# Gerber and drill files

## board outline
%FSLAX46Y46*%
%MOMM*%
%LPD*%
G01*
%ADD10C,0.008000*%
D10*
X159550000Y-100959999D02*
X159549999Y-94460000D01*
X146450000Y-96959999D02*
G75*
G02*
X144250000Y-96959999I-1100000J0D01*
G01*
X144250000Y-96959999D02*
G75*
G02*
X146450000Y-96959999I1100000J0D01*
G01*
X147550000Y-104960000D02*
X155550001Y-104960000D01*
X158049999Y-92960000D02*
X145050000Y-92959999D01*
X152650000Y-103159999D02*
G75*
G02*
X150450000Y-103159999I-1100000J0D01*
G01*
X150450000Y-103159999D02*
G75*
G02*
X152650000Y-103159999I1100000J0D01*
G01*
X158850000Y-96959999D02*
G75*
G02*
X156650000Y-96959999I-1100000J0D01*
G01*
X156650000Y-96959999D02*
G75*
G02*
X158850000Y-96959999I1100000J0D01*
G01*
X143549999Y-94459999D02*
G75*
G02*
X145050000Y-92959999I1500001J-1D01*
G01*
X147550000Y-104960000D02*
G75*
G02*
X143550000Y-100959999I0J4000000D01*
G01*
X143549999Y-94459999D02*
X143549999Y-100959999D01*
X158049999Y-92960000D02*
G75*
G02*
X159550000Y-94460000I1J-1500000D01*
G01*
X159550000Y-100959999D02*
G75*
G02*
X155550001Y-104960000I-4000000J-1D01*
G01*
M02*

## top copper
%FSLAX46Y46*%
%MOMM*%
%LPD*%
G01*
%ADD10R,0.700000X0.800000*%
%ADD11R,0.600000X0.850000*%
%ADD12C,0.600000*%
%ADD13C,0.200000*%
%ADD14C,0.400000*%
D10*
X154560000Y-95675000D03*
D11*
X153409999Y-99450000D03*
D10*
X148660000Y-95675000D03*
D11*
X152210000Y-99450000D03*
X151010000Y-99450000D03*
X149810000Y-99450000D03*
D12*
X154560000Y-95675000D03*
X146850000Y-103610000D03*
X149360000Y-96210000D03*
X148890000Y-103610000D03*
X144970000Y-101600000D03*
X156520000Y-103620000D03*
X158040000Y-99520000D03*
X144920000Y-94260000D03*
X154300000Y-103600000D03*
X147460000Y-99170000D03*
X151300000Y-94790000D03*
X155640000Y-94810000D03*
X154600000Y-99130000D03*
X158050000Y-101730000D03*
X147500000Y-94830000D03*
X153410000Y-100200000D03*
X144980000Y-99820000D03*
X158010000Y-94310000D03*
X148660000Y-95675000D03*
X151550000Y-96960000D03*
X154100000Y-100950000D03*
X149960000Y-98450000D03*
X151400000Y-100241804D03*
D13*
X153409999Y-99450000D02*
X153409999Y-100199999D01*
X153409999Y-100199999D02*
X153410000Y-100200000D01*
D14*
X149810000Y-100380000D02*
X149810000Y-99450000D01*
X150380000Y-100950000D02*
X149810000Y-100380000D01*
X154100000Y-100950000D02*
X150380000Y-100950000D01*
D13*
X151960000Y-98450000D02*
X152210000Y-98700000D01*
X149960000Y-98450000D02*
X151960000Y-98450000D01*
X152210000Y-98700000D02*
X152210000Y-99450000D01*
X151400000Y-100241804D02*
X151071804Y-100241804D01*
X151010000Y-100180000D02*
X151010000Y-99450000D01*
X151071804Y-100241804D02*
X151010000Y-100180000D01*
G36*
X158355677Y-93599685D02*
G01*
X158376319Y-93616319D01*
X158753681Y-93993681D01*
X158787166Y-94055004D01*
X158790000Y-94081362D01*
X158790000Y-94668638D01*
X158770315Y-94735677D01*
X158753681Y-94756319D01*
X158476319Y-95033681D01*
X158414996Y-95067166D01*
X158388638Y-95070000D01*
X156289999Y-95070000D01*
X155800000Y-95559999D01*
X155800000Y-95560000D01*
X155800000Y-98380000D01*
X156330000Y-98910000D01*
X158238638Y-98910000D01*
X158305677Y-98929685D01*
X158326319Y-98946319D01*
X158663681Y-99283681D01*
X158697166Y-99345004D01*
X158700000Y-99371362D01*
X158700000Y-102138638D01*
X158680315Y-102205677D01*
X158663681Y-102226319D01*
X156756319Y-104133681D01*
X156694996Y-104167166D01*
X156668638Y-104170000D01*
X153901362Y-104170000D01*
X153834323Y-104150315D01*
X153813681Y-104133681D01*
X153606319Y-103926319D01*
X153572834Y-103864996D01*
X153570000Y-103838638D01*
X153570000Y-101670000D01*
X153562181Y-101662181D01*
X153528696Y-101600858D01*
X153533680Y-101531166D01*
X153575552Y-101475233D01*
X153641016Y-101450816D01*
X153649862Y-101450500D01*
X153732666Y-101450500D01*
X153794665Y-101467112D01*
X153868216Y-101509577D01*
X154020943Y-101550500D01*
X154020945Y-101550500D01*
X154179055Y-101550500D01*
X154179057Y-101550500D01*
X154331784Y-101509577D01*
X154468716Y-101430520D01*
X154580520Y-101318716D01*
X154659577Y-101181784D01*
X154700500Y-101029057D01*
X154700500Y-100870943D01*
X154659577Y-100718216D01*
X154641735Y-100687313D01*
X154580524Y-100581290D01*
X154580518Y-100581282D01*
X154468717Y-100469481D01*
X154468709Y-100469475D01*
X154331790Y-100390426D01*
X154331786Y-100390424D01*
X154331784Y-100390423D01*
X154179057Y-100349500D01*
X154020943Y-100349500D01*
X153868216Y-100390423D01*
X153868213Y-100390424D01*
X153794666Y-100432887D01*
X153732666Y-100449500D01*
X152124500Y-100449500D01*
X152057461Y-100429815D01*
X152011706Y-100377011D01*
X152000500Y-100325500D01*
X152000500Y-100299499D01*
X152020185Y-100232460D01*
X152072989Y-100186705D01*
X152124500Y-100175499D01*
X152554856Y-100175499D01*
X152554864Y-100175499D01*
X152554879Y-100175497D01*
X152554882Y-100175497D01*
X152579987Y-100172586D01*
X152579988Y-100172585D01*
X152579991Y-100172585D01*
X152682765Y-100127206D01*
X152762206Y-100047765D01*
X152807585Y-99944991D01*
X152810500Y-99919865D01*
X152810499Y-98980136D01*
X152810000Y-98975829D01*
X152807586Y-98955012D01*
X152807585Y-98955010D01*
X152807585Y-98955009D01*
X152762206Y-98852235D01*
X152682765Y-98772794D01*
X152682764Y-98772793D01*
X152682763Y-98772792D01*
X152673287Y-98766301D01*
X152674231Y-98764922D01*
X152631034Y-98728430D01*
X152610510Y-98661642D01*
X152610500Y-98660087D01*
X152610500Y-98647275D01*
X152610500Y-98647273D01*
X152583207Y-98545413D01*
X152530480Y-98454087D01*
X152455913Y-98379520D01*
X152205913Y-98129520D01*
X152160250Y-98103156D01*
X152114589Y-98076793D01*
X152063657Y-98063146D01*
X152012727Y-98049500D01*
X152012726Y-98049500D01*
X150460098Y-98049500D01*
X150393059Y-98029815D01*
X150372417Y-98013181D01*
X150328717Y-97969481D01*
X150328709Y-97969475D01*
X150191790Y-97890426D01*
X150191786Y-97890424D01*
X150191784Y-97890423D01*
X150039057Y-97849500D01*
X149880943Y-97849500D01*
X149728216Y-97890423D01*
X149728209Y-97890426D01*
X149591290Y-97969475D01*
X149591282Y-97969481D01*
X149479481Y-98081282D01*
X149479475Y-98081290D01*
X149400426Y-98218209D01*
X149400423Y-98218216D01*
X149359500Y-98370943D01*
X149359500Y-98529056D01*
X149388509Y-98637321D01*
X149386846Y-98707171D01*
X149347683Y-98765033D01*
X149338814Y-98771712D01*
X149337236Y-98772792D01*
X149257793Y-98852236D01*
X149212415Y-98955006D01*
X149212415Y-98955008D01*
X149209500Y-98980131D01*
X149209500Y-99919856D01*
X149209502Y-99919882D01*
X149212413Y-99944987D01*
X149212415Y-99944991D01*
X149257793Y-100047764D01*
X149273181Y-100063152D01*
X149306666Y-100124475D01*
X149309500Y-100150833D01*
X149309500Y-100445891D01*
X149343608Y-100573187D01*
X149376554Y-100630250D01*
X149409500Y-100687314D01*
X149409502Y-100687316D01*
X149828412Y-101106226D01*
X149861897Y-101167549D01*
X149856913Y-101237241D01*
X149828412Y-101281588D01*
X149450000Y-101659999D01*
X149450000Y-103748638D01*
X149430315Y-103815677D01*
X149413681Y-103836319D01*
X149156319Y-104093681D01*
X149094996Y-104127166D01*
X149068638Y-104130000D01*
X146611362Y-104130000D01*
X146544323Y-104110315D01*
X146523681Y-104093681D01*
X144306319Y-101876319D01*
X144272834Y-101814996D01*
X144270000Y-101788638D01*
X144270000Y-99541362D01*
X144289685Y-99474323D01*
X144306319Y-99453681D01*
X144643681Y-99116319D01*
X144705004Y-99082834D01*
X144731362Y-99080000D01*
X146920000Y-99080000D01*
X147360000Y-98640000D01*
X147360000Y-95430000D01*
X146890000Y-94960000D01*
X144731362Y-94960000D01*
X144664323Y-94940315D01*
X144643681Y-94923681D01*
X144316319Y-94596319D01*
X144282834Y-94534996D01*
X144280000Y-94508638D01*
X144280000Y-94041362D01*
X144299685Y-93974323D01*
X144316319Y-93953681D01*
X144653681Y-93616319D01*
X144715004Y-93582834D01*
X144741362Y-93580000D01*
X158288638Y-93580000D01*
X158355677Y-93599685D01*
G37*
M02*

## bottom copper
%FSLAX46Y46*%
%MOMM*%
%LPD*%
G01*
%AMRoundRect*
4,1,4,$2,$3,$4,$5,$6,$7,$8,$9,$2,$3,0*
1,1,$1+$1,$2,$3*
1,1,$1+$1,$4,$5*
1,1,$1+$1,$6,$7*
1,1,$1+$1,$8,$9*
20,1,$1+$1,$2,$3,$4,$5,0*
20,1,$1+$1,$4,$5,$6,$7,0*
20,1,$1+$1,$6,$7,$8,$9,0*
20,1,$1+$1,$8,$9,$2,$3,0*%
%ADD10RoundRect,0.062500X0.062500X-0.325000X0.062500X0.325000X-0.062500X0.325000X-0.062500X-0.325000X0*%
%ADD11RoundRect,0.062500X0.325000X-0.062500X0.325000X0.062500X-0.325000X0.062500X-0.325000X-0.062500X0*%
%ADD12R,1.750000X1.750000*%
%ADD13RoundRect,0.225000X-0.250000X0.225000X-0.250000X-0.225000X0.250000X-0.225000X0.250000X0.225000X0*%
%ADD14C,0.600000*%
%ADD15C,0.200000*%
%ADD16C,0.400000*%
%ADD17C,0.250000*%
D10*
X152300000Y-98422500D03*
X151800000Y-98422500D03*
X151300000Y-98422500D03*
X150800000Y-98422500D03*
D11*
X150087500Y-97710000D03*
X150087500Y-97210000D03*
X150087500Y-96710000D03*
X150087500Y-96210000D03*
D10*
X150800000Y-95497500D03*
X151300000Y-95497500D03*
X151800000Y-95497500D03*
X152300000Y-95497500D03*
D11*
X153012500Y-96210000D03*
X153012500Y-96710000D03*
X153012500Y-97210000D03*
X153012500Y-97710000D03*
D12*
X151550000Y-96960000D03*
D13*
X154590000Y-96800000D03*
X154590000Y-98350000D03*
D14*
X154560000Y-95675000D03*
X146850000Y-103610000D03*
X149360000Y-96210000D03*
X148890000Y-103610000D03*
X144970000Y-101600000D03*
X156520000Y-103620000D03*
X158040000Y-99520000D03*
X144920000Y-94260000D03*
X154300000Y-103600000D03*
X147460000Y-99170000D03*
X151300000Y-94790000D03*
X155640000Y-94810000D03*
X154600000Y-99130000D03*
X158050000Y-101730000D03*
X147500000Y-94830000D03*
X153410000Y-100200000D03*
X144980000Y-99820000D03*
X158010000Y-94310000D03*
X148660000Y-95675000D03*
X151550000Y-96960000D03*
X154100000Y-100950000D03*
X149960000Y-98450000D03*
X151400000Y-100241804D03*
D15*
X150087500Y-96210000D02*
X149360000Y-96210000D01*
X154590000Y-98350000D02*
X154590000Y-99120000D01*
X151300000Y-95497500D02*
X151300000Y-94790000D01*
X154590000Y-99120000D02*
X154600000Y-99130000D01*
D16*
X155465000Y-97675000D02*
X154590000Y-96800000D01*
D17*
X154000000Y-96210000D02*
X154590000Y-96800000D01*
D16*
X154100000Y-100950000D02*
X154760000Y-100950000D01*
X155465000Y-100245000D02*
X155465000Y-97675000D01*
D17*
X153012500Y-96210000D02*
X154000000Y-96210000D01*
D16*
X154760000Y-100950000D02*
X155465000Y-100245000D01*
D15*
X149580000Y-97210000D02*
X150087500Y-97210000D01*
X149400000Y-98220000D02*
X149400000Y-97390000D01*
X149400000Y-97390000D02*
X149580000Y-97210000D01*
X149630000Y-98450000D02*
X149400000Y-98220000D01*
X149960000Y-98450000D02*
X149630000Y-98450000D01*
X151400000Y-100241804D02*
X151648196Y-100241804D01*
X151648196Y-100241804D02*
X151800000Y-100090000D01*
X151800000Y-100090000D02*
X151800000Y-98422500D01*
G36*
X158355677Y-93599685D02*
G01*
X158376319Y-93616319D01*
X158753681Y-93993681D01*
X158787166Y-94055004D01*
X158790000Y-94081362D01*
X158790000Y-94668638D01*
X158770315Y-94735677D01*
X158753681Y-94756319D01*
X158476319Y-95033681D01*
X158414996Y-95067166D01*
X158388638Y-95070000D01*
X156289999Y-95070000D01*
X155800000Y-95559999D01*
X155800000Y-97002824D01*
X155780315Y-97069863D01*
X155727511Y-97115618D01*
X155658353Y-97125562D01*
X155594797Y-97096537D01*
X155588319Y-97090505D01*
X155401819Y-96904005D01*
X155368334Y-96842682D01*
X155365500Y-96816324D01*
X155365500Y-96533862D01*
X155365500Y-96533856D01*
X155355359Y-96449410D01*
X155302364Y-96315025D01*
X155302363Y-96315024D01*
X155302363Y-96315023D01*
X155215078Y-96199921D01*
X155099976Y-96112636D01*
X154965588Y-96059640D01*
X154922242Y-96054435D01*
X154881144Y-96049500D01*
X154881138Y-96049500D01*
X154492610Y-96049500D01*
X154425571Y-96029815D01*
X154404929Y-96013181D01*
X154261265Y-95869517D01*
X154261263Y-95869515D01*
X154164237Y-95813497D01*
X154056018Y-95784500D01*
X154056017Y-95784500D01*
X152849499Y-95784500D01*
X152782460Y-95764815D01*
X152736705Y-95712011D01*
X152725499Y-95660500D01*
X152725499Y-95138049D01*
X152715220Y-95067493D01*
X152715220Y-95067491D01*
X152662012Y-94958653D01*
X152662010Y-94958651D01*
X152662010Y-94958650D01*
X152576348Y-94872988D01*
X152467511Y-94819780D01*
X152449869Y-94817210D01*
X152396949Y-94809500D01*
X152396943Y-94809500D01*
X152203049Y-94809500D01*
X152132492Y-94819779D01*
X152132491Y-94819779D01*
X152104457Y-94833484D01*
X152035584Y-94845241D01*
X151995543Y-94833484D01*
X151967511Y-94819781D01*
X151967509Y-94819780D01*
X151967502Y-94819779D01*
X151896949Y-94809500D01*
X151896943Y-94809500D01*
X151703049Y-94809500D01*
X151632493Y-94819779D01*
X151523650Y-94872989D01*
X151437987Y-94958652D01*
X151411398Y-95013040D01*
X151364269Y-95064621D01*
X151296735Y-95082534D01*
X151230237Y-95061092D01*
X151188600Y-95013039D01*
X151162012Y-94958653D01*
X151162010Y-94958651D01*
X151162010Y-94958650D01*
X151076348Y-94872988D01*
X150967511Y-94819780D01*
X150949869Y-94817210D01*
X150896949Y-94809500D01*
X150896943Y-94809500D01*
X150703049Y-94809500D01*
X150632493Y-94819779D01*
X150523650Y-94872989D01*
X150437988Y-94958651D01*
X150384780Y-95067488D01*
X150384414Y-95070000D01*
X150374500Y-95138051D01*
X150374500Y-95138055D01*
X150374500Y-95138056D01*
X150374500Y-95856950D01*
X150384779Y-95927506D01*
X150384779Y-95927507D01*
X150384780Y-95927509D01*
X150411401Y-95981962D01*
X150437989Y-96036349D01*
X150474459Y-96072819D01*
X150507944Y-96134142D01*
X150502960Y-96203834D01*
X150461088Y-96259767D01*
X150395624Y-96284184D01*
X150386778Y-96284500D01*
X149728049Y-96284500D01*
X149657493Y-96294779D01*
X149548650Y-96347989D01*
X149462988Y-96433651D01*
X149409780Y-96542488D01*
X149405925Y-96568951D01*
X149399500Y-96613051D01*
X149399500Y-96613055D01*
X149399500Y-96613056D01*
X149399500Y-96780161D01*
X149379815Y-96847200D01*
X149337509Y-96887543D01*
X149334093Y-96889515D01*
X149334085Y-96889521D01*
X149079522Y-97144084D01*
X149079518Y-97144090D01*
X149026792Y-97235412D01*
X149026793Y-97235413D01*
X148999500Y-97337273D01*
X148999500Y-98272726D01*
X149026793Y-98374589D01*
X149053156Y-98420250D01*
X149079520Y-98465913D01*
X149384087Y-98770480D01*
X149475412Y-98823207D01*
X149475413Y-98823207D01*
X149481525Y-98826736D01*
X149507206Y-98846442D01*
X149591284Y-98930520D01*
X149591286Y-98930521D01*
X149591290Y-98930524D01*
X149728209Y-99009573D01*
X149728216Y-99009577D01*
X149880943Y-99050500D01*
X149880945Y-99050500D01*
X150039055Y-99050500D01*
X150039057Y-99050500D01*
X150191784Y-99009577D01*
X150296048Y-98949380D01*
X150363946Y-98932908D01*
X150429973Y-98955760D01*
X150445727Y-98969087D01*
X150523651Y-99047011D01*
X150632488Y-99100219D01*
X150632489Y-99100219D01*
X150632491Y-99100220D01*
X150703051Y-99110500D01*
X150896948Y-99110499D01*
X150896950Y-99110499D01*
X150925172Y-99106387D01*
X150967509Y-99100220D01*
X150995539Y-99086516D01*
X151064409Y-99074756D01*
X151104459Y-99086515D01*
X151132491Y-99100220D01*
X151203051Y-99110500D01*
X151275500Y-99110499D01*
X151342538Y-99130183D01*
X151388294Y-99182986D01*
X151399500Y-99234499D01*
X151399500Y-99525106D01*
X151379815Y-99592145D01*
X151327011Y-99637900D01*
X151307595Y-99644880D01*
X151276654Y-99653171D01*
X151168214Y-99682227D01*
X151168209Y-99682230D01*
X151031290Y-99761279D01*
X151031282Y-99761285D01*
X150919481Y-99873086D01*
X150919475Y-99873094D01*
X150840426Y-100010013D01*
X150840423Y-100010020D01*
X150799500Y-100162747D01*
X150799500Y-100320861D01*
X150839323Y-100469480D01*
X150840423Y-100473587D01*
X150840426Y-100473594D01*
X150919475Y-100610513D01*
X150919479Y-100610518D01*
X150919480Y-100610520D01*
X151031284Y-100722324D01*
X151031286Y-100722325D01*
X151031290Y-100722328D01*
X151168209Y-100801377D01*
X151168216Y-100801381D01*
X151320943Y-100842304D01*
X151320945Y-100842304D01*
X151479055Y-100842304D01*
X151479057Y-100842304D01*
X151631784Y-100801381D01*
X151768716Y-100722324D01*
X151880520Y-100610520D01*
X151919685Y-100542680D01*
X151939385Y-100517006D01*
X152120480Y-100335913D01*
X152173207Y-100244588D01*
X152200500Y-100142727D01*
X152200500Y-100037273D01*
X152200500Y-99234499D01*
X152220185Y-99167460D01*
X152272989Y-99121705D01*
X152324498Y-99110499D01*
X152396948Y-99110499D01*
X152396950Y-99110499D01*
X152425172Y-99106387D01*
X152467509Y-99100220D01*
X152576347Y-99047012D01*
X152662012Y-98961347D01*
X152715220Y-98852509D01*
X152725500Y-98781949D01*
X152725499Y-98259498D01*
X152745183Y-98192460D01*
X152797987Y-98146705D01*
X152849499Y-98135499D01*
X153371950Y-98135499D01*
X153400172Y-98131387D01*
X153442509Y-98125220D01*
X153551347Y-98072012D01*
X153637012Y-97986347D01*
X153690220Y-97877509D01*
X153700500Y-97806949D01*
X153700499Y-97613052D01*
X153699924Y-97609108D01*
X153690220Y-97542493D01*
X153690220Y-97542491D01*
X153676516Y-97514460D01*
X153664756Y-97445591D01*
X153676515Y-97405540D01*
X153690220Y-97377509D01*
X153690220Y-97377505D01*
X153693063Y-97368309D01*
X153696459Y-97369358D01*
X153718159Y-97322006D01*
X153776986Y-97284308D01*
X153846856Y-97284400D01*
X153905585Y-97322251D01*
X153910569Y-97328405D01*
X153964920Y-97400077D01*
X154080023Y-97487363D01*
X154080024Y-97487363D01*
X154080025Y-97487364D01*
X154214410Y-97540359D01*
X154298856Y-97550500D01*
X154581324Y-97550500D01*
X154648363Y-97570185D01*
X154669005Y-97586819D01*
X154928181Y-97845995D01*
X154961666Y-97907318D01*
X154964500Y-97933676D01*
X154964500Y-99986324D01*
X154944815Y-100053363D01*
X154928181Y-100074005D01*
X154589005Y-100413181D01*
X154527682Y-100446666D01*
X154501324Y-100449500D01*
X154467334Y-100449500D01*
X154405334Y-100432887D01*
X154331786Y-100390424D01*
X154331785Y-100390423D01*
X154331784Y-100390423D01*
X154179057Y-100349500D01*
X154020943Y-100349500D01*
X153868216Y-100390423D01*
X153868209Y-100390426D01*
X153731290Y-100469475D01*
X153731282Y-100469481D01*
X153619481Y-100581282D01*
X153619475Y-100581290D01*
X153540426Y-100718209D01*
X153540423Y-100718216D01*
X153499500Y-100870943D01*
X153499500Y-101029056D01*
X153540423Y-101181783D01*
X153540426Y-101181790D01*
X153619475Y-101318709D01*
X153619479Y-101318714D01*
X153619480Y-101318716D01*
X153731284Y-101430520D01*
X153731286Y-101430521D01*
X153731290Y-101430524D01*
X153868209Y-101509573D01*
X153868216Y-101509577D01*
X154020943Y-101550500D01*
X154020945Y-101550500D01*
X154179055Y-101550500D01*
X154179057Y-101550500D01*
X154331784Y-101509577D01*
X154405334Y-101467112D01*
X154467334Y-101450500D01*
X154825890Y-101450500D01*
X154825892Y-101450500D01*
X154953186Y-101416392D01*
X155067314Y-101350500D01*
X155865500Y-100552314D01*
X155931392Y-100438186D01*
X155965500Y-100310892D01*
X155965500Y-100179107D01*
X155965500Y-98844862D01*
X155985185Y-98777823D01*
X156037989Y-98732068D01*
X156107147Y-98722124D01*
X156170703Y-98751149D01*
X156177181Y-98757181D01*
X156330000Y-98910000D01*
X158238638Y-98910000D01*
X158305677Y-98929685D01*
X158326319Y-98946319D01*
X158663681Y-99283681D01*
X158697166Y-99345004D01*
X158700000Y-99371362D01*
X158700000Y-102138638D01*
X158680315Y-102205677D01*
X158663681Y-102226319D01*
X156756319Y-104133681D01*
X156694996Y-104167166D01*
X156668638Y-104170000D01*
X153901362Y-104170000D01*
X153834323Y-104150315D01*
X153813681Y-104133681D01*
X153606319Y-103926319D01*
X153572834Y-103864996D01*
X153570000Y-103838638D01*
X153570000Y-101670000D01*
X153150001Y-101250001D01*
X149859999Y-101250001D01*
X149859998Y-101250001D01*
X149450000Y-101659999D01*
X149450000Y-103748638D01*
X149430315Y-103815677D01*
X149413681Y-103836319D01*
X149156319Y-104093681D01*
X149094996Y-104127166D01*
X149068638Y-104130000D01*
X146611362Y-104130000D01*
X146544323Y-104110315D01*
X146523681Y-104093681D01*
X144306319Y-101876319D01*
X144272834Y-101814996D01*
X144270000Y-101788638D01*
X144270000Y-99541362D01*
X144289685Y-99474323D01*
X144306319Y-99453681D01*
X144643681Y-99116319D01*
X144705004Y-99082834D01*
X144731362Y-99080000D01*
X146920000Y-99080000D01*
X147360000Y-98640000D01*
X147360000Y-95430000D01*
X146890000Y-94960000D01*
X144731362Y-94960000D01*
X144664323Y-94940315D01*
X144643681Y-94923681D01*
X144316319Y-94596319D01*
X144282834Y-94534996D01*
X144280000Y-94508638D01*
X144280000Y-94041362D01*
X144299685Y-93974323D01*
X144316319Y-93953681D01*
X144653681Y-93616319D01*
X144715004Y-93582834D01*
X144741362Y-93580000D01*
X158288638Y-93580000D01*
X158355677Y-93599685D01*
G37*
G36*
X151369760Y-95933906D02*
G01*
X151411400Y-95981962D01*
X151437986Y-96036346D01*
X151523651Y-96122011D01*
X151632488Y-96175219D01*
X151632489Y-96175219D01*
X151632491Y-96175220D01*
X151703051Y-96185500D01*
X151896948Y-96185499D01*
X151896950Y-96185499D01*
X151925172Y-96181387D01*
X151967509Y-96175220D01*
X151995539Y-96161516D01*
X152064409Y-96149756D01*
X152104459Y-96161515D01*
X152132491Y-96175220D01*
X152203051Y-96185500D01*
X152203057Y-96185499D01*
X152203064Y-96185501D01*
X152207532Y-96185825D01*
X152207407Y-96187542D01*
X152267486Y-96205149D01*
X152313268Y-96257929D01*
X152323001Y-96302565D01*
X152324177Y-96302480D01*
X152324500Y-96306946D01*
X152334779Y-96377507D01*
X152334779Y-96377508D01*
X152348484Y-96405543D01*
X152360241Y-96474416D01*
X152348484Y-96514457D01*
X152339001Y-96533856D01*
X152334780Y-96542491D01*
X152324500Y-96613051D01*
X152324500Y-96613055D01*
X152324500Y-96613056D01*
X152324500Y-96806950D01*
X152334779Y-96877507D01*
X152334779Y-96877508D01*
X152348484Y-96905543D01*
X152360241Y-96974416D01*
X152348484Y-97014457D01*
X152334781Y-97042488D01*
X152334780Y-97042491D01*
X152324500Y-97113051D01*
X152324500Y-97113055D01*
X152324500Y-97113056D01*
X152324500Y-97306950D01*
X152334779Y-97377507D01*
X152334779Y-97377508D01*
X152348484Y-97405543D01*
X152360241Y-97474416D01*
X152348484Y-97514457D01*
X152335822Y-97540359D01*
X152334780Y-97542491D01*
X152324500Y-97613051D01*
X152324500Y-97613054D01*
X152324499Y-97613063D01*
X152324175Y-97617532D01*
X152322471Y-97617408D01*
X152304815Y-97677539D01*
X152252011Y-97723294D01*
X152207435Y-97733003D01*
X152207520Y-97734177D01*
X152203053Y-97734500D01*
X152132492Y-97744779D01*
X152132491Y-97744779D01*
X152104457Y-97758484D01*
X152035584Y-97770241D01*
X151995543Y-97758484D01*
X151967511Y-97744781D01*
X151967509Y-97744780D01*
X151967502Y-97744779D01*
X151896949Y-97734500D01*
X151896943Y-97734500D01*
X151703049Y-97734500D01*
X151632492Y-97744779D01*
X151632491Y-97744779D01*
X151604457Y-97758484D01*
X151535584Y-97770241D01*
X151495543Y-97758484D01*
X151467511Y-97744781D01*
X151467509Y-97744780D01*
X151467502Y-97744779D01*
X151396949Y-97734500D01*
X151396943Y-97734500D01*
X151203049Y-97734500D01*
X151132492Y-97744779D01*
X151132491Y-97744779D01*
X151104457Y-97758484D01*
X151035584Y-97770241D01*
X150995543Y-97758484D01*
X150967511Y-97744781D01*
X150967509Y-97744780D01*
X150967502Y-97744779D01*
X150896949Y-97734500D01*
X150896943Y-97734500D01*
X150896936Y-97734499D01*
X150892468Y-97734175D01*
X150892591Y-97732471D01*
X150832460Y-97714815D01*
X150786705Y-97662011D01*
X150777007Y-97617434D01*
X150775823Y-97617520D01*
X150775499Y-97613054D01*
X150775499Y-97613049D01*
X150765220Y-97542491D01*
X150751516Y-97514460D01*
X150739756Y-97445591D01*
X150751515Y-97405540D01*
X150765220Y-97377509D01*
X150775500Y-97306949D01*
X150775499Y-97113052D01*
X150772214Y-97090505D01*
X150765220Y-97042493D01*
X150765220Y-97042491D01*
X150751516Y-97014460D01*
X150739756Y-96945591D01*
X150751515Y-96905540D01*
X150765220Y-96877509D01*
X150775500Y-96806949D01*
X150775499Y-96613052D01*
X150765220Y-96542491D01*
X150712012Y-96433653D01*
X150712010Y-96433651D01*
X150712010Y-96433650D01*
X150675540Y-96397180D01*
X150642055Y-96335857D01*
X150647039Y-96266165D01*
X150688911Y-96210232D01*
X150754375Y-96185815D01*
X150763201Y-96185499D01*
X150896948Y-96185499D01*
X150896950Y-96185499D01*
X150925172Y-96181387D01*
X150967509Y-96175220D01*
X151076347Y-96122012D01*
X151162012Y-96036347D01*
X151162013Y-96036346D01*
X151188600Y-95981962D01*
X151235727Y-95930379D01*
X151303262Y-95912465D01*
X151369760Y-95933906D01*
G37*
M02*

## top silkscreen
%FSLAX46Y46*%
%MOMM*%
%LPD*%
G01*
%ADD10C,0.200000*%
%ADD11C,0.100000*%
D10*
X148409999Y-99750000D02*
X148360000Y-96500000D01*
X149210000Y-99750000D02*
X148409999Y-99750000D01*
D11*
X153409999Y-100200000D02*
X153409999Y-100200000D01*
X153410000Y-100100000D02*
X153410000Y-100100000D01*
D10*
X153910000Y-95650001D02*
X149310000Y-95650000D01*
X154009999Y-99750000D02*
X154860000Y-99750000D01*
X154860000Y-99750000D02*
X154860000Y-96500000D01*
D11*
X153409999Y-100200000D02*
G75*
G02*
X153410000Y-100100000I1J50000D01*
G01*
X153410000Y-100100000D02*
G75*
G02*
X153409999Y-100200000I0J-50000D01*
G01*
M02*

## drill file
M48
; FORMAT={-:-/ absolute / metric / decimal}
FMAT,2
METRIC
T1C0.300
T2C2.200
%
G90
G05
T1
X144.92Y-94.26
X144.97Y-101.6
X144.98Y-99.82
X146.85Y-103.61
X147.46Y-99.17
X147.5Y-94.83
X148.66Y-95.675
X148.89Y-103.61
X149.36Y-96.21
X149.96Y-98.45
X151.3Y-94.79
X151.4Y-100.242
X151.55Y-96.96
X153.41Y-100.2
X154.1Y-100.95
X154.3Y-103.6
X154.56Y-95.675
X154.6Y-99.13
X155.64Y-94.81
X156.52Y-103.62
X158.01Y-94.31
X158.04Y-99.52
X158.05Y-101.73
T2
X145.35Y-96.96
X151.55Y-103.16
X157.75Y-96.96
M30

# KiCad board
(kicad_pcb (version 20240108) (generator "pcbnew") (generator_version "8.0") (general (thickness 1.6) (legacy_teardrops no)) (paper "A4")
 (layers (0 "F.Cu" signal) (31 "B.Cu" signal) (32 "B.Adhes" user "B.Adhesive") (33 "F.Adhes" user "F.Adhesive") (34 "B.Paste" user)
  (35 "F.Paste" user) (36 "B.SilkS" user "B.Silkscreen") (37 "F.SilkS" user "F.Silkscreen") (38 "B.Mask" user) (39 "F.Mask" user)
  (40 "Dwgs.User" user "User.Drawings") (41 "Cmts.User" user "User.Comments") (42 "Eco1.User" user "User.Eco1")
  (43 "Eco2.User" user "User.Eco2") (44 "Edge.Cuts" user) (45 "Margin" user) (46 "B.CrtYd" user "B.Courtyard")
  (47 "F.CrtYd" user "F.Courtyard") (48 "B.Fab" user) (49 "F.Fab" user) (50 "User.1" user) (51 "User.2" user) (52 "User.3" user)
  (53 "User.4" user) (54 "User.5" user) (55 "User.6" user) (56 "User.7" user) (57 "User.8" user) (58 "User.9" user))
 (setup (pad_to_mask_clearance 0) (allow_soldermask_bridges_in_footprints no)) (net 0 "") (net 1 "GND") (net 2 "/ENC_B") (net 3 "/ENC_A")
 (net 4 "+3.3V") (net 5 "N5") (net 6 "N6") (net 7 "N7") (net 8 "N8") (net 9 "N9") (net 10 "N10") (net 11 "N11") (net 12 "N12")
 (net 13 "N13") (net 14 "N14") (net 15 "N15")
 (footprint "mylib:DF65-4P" (layer "F.Cu") (at 151.585 97.800001 180)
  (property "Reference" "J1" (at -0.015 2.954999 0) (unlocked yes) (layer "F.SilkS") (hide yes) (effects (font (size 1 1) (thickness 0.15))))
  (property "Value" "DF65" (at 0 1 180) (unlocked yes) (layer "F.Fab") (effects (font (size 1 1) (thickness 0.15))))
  (fp_line (start 3.175001 -1.949999) (end 3.225 1.300001) (stroke (width 0.2) (type solid)) (layer "F.SilkS"))
  (fp_line (start 2.375 -1.949999) (end 3.175001 -1.949999) (stroke (width 0.2) (type solid)) (layer "F.SilkS"))
  (fp_line (start -1.824999 -2.399999) (end -1.824999 -2.399999) (stroke (width 0.1) (type solid)) (layer "F.SilkS"))
  (fp_line (start -1.825 -2.299999) (end -1.825 -2.299999) (stroke (width 0.1) (type solid)) (layer "F.SilkS"))
  (fp_line (start -2.325 2.15) (end 2.275 2.150001) (stroke (width 0.2) (type solid)) (layer "F.SilkS"))
  (fp_line (start -2.424999 -1.949999) (end -3.275 -1.949999) (stroke (width 0.2) (type solid)) (layer "F.SilkS"))
  (fp_line (start -3.275 -1.949999) (end -3.275 1.300001) (stroke (width 0.2) (type solid)) (layer "F.SilkS"))
  (fp_arc (start -1.824999 -2.399999) (mid -1.775 -2.349998) (end -1.825 -2.299999) (stroke (width 0.1) (type solid)) (layer "F.SilkS"))
  (fp_arc (start -1.825 -2.299999) (mid -1.875 -2.349999) (end -1.824999 -2.399999) (stroke (width 0.1) (type solid)) (layer "F.SilkS"))
  (pad "1" smd rect (at -2.975 2.125001 180) (size 0.7 0.8) (layers "F.Cu" "F.Paste" "F.Mask") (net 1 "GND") (thermal_bridge_angle 45))
  (pad "1" smd rect (at -1.824999 -1.649999 180) (size 0.6 0.85) (layers "F.Cu" "F.Paste" "F.Mask") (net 1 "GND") (thermal_bridge_angle 45))
  (pad "1" smd rect (at 2.925 2.125001 180) (size 0.7 0.8) (layers "F.Cu" "F.Paste" "F.Mask") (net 1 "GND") (thermal_bridge_angle 45))
  (pad "2" smd rect (at -0.625 -1.649999 180) (size 0.6 0.85) (layers "F.Cu" "F.Paste" "F.Mask") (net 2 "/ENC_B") (thermal_bridge_angle 45))
  (pad "3" smd rect (at 0.575 -1.649999 180) (size 0.6 0.85) (layers "F.Cu" "F.Paste" "F.Mask") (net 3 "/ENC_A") (thermal_bridge_angle 45))
  (pad "4" smd rect (at 1.775 -1.649999 180) (size 0.6 0.85) (layers "F.Cu" "F.Paste" "F.Mask") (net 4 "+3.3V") (thermal_bridge_angle 45)))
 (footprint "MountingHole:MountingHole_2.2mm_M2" (layer "F.Cu") (at 145.35 96.959999)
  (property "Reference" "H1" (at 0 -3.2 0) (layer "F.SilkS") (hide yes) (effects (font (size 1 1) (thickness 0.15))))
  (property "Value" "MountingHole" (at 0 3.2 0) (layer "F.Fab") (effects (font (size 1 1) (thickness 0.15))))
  (pad "" np_thru_hole circle (at 0 0) (size 2.2 2.2) (drill 2.2) (layers "*.Cu" "*.Mask")))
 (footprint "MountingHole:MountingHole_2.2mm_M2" (layer "F.Cu") (at 157.75 96.959999)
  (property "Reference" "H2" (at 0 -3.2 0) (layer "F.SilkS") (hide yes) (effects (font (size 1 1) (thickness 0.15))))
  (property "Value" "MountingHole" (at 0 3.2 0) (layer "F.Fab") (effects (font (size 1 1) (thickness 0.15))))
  (pad "" np_thru_hole circle (at 0 0) (size 2.2 2.2) (drill 2.2) (layers "*.Cu" "*.Mask")))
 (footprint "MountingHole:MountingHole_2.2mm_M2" (layer "F.Cu") (at 151.55 103.159999)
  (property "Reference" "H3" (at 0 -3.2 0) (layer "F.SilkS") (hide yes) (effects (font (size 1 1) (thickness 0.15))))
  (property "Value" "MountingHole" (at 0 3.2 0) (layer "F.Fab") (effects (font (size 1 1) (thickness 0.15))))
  (pad "" np_thru_hole circle (at 0 0) (size 2.2 2.2) (drill 2.2) (layers "*.Cu" "*.Mask")))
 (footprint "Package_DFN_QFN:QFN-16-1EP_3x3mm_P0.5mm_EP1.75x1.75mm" (layer "B.Cu") (at 151.55 96.96 90)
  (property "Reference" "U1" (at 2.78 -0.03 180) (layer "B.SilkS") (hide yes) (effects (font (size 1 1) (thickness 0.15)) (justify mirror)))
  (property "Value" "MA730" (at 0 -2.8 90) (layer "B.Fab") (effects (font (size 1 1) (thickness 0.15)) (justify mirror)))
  (pad "" smd roundrect (at -0.44 -0.44 90) (size 0.71 0.71) (layers "B.Paste") (roundrect_rratio 0.25))
  (pad "" smd roundrect (at -0.44 0.44 90) (size 0.71 0.71) (layers "B.Paste") (roundrect_rratio 0.25))
  (pad "" smd roundrect (at 0.44 -0.44 90) (size 0.71 0.71) (layers "B.Paste") (roundrect_rratio 0.25))
  (pad "" smd roundrect (at 0.44 0.44 90) (size 0.71 0.71) (layers "B.Paste") (roundrect_rratio 0.25))
  (pad "1" smd roundrect (at -1.4625 0.75 90) (size 0.775 0.25) (layers "B.Cu" "B.Paste" "B.Mask") (roundrect_rratio 0.25) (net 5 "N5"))
  (pad "2" smd roundrect (at -1.4625 0.25 90) (size 0.775 0.25) (layers "B.Cu" "B.Paste" "B.Mask") (roundrect_rratio 0.25) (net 3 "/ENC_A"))
  (pad "3" smd roundrect (at -1.4625 -0.25 90) (size 0.775 0.25) (layers "B.Cu" "B.Paste" "B.Mask") (roundrect_rratio 0.25) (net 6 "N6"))
  (pad "4" smd roundrect (at -1.4625 -0.75 90) (size 0.775 0.25) (layers "B.Cu" "B.Paste" "B.Mask") (roundrect_rratio 0.25) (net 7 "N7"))
  (pad "5" smd roundrect (at -0.75 -1.4625 90) (size 0.25 0.775) (layers "B.Cu" "B.Paste" "B.Mask") (roundrect_rratio 0.25) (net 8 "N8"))
  (pad "6" smd roundrect (at -0.25 -1.4625 90) (size 0.25 0.775) (layers "B.Cu" "B.Paste" "B.Mask") (roundrect_rratio 0.25) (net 2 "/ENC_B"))
  (pad "7" smd roundrect (at 0.25 -1.4625 90) (size 0.25 0.775) (layers "B.Cu" "B.Paste" "B.Mask") (roundrect_rratio 0.25) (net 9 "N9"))
  (pad "8" smd roundrect (at 0.75 -1.4625 90) (size 0.25 0.775) (layers "B.Cu" "B.Paste" "B.Mask") (roundrect_rratio 0.25) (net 1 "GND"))
  (pad "9" smd roundrect (at 1.4625 -0.75 90) (size 0.775 0.25) (layers "B.Cu" "B.Paste" "B.Mask") (roundrect_rratio 0.25) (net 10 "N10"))
  (pad "10" smd roundrect (at 1.4625 -0.25 90) (size 0.775 0.25) (layers "B.Cu" "B.Paste" "B.Mask") (roundrect_rratio 0.25) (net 1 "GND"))
  (pad "11" smd roundrect (at 1.4625 0.25 90) (size 0.775 0.25) (layers "B.Cu" "B.Paste" "B.Mask") (roundrect_rratio 0.25) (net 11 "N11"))
  (pad "12" smd roundrect (at 1.4625 0.75 90) (size 0.775 0.25) (layers "B.Cu" "B.Paste" "B.Mask") (roundrect_rratio 0.25) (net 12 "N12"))
  (pad "13" smd roundrect (at 0.75 1.4625 90) (size 0.25 0.775) (layers "B.Cu" "B.Paste" "B.Mask") (roundrect_rratio 0.25) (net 4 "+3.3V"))
  (pad "14" smd roundrect (at 0.25 1.4625 90) (size 0.25 0.775) (layers "B.Cu" "B.Paste" "B.Mask") (roundrect_rratio 0.25) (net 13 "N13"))
  (pad "15" smd roundrect (at -0.25 1.4625 90) (size 0.25 0.775) (layers "B.Cu" "B.Paste" "B.Mask") (roundrect_rratio 0.25) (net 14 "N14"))
  (pad "16" smd roundrect (at -0.75 1.4625 90) (size 0.25 0.775) (layers "B.Cu" "B.Paste" "B.Mask") (roundrect_rratio 0.25) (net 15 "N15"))
  (pad "17" smd rect (at 0 0 90) (size 1.75 1.75) (layers "B.Cu" "B.Mask") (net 1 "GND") (zone_connect 2)))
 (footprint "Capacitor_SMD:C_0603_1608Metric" (layer "B.Cu") (at 154.59 97.575 -90)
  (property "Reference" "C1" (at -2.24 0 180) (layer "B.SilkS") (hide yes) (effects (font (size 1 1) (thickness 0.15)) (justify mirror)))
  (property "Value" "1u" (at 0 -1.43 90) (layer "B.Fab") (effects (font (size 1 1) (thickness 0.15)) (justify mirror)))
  (pad "1" smd roundrect (at -0.775 0 270) (size 0.9 0.95) (layers "B.Cu" "B.Paste" "B.Mask") (roundrect_rratio 0.25) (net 4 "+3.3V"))
  (pad "2" smd roundrect (at 0.775 0 270) (size 0.9 0.95) (layers "B.Cu" "B.Paste" "B.Mask") (roundrect_rratio 0.25) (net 1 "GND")))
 (gr_line (start 159.55 100.959999) (end 159.549999 94.46) (stroke (width 0.008) (type default)) (layer "Edge.Cuts"))
 (gr_circle (center 145.35 96.959999) (end 144.25 96.959999) (stroke (width 0.008) (type default)) (fill none) (layer "Edge.Cuts"))
 (gr_line (start 147.55 104.96) (end 155.550001 104.96) (stroke (width 0.008) (type default)) (layer "Edge.Cuts"))
 (gr_line (start 158.049999 92.96) (end 145.05 92.959999) (stroke (width 0.008) (type default)) (layer "Edge.Cuts"))
 (gr_circle (center 151.55 103.159999) (end 150.45 103.159999) (stroke (width 0.008) (type default)) (fill none) (layer "Edge.Cuts"))
 (gr_circle (center 157.75 96.959999) (end 156.65 96.959999) (stroke (width 0.008) (type default)) (fill none) (layer "Edge.Cuts"))
 (gr_arc (start 143.549999 94.459999) (mid 143.989339 93.399338) (end 145.05 92.959999) (stroke (width 0.008) (type default))
  (layer "Edge.Cuts"))
 (gr_arc (start 147.55 104.96) (mid 144.721572 103.788427) (end 143.549999 100.959999) (stroke (width 0.008) (type default))
  (layer "Edge.Cuts"))
 (gr_line (start 143.549999 94.459999) (end 143.549999 100.959999) (stroke (width 0.008) (type default)) (layer "Edge.Cuts"))
 (gr_arc (start 158.049999 92.96) (mid 159.11066 93.39934) (end 159.549999 94.46) (stroke (width 0.008) (type default)) (layer "Edge.Cuts"))
 (gr_arc (start 159.55 100.959999) (mid 158.378427 103.788426) (end 155.550001 104.96) (stroke (width 0.008) (type default))
  (layer "Edge.Cuts"))
 (segment (start 153.409999 99.45) (end 153.409999 100.199999) (width 0.2) (layer "F.Cu") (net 1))
 (segment (start 153.409999 100.199999) (end 153.41 100.2) (width 0.2) (layer "F.Cu") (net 1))
 (via (at 154.56 95.675) (size 0.6) (drill 0.3) (layers "F.Cu" "B.Cu") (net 1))
 (via (at 146.85 103.61) (size 0.6) (drill 0.3) (layers "F.Cu" "B.Cu") (free yes) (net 1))
 (via (at 149.36 96.21) (size 0.6) (drill 0.3) (layers "F.Cu" "B.Cu") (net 1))
 (via (at 148.89 103.61) (size 0.6) (drill 0.3) (layers "F.Cu" "B.Cu") (free yes) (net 1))
 (via (at 144.97 101.6) (size 0.6) (drill 0.3) (layers "F.Cu" "B.Cu") (free yes) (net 1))
 (via (at 156.52 103.62) (size 0.6) (drill 0.3) (layers "F.Cu" "B.Cu") (free yes) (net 1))
 (via (at 158.04 99.52) (size 0.6) (drill 0.3) (layers "F.Cu" "B.Cu") (free yes) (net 1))
 (via (at 144.92 94.26) (size 0.6) (drill 0.3) (layers "F.Cu" "B.Cu") (free yes) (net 1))
 (via (at 154.3 103.6) (size 0.6) (drill 0.3) (layers "F.Cu" "B.Cu") (free yes) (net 1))
 (via (at 147.46 99.17) (size 0.6) (drill 0.3) (layers "F.Cu" "B.Cu") (free yes) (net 1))
 (via (at 151.3 94.79) (size 0.6) (drill 0.3) (layers "F.Cu" "B.Cu") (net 1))
 (via (at 155.64 94.81) (size 0.6) (drill 0.3) (layers "F.Cu" "B.Cu") (free yes) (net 1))
 (via (at 154.6 99.13) (size 0.6) (drill 0.3) (layers "F.Cu" "B.Cu") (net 1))
 (via (at 158.05 101.73) (size 0.6) (drill 0.3) (layers "F.Cu" "B.Cu") (free yes) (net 1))
 (via (at 147.5 94.83) (size 0.6) (drill 0.3) (layers "F.Cu" "B.Cu") (free yes) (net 1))
 (via (at 153.41 100.2) (size 0.6) (drill 0.3) (layers "F.Cu" "B.Cu") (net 1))
 (via (at 144.98 99.82) (size 0.6) (drill 0.3) (layers "F.Cu" "B.Cu") (free yes) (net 1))
 (via (at 158.01 94.31) (size 0.6) (drill 0.3) (layers "F.Cu" "B.Cu") (free yes) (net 1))
 (via (at 148.66 95.675) (size 0.6) (drill 0.3) (layers "F.Cu" "B.Cu") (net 1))
 (via (at 151.55 96.96) (size 0.6) (drill 0.3) (layers "F.Cu" "B.Cu") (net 1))
 (segment (start 150.0875 96.21) (end 149.36 96.21) (width 0.2) (layer "B.Cu") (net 1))
 (segment (start 154.59 98.35) (end 154.59 99.12) (width 0.2) (layer "B.Cu") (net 1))
 (segment (start 151.3 95.4975) (end 151.3 94.79) (width 0.2) (layer "B.Cu") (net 1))
 (segment (start 154.59 99.12) (end 154.6 99.13) (width 0.2) (layer "B.Cu") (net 1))
 (segment (start 149.81 100.38) (end 149.81 99.45) (width 0.4) (layer "F.Cu") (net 4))
 (segment (start 150.38 100.95) (end 149.81 100.38) (width 0.4) (layer "F.Cu") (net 4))
 (segment (start 154.1 100.95) (end 150.38 100.95) (width 0.4) (layer "F.Cu") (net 4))
 (via (at 154.1 100.95) (size 0.6) (drill 0.3) (layers "F.Cu" "B.Cu") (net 4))
 (segment (start 155.465 97.675) (end 154.59 96.8) (width 0.4) (layer "B.Cu") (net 4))
 (segment (start 154 96.21) (end 154.59 96.8) (width 0.25) (layer "B.Cu") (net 4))
 (segment (start 154.1 100.95) (end 154.76 100.95) (width 0.4) (layer "B.Cu") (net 4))
 (segment (start 155.465 100.245) (end 155.465 97.675) (width 0.4) (layer "B.Cu") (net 4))
 (segment (start 153.0125 96.21) (end 154 96.21) (width 0.25) (layer "B.Cu") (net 4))
 (segment (start 154.76 100.95) (end 155.465 100.245) (width 0.4) (layer "B.Cu") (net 4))
 (segment (start 151.96 98.45) (end 152.21 98.7) (width 0.2) (layer "F.Cu") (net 2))
 (segment (start 149.96 98.45) (end 151.96 98.45) (width 0.2) (layer "F.Cu") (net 2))
 (segment (start 152.21 98.7) (end 152.21 99.45) (width 0.2) (layer "F.Cu") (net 2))
 (via (at 149.96 98.45) (size 0.6) (drill 0.3) (layers "F.Cu" "B.Cu") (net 2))
 (segment (start 149.58 97.21) (end 150.0875 97.21) (width 0.2) (layer "B.Cu") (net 2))
 (segment (start 149.4 98.22) (end 149.4 97.39) (width 0.2) (layer "B.Cu") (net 2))
 (segment (start 149.4 97.39) (end 149.58 97.21) (width 0.2) (layer "B.Cu") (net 2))
 (segment (start 149.63 98.45) (end 149.4 98.22) (width 0.2) (layer "B.Cu") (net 2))
 (segment (start 149.96 98.45) (end 149.63 98.45) (width 0.2) (layer "B.Cu") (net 2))
 (segment (start 151.4 100.241804) (end 151.071804 100.241804) (width 0.2) (layer "F.Cu") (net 3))
 (segment (start 151.01 100.18) (end 151.01 99.45) (width 0.2) (layer "F.Cu") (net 3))
 (segment (start 151.071804 100.241804) (end 151.01 100.18) (width 0.2) (layer "F.Cu") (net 3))
 (via (at 151.4 100.241804) (size 0.6) (drill 0.3) (layers "F.Cu" "B.Cu") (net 3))
 (segment (start 151.4 100.241804) (end 151.648196 100.241804) (width 0.2) (layer "B.Cu") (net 3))
 (segment (start 151.648196 100.241804) (end 151.8 100.09) (width 0.2) (layer "B.Cu") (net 3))
 (segment (start 151.8 100.09) (end 151.8 98.4225) (width 0.2) (layer "B.Cu") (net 3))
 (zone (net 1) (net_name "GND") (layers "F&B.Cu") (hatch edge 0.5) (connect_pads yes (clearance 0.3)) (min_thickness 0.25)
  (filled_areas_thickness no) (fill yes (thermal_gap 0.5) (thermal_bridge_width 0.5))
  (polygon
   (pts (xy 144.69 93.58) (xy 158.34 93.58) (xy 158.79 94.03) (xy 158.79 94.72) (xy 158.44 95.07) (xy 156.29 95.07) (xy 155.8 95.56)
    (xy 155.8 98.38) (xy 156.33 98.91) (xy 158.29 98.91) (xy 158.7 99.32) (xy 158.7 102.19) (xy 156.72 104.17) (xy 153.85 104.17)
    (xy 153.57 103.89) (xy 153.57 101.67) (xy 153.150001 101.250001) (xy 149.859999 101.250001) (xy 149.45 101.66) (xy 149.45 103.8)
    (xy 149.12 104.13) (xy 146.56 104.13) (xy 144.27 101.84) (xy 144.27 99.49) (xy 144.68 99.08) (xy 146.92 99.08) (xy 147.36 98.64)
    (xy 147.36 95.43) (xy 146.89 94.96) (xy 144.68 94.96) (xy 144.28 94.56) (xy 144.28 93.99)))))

